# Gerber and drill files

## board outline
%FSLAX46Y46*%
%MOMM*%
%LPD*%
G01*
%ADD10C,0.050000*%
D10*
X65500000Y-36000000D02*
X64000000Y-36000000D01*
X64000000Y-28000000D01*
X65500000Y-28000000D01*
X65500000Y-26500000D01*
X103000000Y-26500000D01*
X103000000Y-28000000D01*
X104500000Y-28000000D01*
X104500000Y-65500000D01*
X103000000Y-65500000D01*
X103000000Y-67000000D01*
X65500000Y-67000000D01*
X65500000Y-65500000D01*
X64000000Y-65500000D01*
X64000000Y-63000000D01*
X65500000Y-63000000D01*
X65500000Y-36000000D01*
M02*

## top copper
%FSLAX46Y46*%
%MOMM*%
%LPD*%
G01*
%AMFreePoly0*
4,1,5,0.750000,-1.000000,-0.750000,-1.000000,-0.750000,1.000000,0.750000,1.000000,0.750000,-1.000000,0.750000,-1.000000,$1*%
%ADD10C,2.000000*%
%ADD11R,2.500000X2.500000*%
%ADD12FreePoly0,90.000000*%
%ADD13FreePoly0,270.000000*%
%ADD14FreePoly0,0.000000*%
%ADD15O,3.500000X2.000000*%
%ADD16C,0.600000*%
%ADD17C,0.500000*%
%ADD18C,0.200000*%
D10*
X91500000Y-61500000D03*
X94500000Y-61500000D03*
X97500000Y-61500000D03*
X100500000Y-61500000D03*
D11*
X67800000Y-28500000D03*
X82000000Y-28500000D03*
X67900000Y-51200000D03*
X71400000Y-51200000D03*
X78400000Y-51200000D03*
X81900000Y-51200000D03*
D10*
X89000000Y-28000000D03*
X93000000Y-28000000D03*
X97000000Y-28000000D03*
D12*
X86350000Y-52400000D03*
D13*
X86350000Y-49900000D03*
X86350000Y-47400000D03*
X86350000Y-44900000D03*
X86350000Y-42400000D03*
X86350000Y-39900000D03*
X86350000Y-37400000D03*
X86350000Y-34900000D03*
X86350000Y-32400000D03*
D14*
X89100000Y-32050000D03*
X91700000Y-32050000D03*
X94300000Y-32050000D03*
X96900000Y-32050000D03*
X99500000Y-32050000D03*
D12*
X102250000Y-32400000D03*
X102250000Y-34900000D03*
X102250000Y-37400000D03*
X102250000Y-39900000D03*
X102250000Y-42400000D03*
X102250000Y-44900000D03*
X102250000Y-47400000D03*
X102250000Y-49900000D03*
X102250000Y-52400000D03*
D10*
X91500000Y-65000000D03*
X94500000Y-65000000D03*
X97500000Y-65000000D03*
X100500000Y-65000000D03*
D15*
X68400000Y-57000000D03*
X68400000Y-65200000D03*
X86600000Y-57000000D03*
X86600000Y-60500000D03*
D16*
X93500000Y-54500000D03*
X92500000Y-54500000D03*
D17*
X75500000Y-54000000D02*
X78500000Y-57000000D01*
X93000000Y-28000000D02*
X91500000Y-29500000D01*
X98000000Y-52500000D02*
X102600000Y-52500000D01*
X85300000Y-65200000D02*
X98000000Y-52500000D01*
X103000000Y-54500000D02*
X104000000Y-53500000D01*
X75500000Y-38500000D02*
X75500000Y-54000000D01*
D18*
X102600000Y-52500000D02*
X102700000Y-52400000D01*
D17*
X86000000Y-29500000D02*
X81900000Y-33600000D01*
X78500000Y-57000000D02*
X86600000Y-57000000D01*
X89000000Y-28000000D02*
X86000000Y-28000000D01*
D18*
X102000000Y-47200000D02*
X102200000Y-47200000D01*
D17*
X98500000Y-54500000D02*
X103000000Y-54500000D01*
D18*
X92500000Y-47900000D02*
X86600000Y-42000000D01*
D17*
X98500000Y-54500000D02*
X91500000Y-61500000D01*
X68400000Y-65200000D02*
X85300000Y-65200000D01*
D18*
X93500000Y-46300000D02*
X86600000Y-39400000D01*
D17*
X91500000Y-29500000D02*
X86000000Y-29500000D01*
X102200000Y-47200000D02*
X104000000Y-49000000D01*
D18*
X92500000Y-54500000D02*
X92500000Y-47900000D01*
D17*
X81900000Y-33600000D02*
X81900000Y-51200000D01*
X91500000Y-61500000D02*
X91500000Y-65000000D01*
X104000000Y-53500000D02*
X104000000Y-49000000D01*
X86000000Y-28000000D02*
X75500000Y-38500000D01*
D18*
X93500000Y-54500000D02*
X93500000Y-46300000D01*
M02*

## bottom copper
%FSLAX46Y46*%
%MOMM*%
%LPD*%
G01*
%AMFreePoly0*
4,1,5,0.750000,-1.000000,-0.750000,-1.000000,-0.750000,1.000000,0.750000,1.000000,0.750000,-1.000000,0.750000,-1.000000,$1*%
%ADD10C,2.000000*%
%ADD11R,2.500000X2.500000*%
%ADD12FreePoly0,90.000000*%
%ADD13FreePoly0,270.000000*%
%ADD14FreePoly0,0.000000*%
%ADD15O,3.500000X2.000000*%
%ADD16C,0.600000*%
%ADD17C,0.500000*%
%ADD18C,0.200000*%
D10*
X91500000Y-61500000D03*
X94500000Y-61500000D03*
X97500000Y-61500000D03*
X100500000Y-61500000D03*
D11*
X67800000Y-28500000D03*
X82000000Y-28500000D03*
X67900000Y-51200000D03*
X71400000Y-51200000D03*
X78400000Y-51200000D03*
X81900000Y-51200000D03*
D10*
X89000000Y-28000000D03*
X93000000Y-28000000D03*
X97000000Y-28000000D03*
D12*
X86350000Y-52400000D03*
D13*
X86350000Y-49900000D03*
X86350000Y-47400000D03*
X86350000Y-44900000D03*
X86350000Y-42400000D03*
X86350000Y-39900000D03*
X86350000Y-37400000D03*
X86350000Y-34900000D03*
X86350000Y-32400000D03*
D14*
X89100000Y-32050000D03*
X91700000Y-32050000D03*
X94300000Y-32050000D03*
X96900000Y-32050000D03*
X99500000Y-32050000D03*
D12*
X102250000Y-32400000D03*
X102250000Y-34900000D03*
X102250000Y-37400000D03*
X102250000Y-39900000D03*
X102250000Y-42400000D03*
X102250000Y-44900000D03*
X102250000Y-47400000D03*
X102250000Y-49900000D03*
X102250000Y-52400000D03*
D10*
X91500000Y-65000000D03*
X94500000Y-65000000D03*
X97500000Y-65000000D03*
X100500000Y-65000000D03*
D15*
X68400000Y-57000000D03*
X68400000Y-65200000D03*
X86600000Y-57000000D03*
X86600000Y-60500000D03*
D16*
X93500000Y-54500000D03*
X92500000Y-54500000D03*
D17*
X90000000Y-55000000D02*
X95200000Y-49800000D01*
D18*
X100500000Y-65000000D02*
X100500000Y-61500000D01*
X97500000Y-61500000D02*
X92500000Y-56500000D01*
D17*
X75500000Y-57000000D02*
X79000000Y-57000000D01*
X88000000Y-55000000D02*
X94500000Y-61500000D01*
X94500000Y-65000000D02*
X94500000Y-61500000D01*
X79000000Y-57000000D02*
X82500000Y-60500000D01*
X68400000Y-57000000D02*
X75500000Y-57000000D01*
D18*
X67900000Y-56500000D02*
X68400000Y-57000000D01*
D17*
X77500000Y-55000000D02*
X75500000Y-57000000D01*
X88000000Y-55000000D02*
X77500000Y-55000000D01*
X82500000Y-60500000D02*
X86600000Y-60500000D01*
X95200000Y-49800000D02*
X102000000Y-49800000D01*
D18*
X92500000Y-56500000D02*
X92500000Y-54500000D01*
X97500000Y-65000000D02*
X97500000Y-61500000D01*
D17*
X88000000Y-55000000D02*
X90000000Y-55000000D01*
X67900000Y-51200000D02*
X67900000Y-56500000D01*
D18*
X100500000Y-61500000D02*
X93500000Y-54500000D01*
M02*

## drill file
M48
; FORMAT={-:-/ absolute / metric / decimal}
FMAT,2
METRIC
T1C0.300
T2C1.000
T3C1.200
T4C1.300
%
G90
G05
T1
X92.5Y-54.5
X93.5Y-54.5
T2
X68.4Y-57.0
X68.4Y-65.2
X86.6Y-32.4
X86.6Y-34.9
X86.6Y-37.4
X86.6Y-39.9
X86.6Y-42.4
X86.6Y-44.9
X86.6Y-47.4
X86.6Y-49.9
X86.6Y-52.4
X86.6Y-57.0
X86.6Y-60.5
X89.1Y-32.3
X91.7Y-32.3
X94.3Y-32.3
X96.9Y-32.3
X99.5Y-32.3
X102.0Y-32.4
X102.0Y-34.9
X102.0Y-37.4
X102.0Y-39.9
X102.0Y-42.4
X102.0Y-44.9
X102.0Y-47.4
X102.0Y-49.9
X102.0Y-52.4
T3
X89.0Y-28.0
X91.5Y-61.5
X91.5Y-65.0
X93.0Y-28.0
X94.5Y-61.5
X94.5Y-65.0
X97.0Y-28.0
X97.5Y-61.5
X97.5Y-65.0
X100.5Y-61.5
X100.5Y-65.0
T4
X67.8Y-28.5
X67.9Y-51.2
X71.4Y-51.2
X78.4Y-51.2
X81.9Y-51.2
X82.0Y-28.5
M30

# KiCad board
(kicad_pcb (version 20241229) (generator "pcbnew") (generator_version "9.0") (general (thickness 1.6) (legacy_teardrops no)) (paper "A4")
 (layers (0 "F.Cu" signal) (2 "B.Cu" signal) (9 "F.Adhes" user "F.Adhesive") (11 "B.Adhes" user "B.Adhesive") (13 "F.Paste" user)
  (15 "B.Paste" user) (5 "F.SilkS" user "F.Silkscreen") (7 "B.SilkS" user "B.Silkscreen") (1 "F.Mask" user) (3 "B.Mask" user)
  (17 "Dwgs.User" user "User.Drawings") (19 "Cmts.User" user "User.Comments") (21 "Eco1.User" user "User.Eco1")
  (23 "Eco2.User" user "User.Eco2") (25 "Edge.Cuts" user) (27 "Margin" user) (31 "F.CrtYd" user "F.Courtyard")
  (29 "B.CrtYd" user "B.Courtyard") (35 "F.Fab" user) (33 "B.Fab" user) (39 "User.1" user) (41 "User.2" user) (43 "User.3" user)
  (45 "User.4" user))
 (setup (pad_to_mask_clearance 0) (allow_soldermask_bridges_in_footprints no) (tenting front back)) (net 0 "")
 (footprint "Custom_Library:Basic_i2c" (layer "F.Cu") (at 96 61.5)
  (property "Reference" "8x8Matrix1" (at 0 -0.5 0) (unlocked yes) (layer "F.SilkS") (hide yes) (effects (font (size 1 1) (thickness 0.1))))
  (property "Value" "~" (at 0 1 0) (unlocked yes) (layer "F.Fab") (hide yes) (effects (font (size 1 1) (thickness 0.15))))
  (pad "1" thru_hole circle (at -4.5 0) (size 2 2) (drill 1.2) (layers "*.Cu" "*.Mask") (remove_unused_layers no))
  (pad "2" thru_hole circle (at -1.5 0) (size 2 2) (drill 1.2) (layers "*.Cu" "*.Mask") (remove_unused_layers no))
  (pad "3" thru_hole circle (at 1.5 0) (size 2 2) (drill 1.2) (layers "*.Cu" "*.Mask") (remove_unused_layers no))
  (pad "4" thru_hole circle (at 4.5 0) (size 2 2) (drill 1.2) (layers "*.Cu" "*.Mask") (remove_unused_layers no)))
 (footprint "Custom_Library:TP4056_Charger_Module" (layer "F.Cu") (at 74.9 41)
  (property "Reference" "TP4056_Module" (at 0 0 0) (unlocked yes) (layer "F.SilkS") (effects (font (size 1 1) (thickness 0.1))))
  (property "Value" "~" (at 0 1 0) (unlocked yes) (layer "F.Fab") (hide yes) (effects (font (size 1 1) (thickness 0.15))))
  (pad "1" thru_hole rect (at -7.1 -12.5) (size 2.5 2.5) (drill 1.3) (layers "*.Cu" "*.Mask") (remove_unused_layers no)
   (thermal_bridge_angle 45))
  (pad "2" thru_hole rect (at 7.1 -12.5) (size 2.5 2.5) (drill 1.3) (layers "*.Cu" "*.Mask") (remove_unused_layers no)
   (thermal_bridge_angle 45))
  (pad "3" thru_hole rect (at -7 10.2) (size 2.5 2.5) (drill 1.3) (layers "*.Cu" "*.Mask") (remove_unused_layers no)
   (thermal_bridge_angle 45))
  (pad "4" thru_hole rect (at -3.5 10.2) (size 2.5 2.5) (drill 1.3) (layers "*.Cu" "*.Mask") (remove_unused_layers no)
   (thermal_bridge_angle 45))
  (pad "5" thru_hole rect (at 3.5 10.2) (size 2.5 2.5) (drill 1.3) (layers "*.Cu" "*.Mask") (remove_unused_layers no)
   (thermal_bridge_angle 45))
  (pad "6" thru_hole rect (at 7 10.2) (size 2.5 2.5) (drill 1.3) (layers "*.Cu" "*.Mask") (remove_unused_layers no)
   (thermal_bridge_angle 45)))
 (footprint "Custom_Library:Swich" (layer "F.Cu") (at 93 28)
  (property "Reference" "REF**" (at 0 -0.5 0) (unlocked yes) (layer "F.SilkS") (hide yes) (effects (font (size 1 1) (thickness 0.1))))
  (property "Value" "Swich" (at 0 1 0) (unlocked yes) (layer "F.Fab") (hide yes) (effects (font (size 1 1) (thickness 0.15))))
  (pad "1" thru_hole circle (at -4 0) (size 2 2) (drill 1.2) (layers "*.Cu" "*.Mask") (remove_unused_layers no))
  (pad "2" thru_hole circle (at 0 0) (size 2 2) (drill 1.2) (layers "*.Cu" "*.Mask") (remove_unused_layers no))
  (pad "3" thru_hole circle (at 4 0) (size 2 2) (drill 1.2) (layers "*.Cu" "*.Mask") (remove_unused_layers no)))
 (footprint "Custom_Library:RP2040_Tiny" (layer "F.Cu") (at 94.3 42 90)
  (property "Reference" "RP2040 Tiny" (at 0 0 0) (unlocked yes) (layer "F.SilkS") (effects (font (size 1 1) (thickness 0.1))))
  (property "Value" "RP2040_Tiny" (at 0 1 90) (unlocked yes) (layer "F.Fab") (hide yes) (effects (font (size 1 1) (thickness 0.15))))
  (pad "1" thru_hole custom (at -10.4 -7.7 90) (size 1.5 2) (drill 1 (offset 0 -0.25)) (layers "*.Cu" "*.Mask") (remove_unused_layers no)
   (options (clearance outline) (anchor rect)) (primitives))
  (pad "2" thru_hole custom (at -7.9 -7.7 270) (size 1.5 2) (drill 1 (offset 0 0.25)) (layers "*.Cu" "*.Mask") (remove_unused_layers no)
   (options (clearance outline) (anchor rect)) (primitives))
  (pad "3" thru_hole custom (at -5.4 -7.7 270) (size 1.5 2) (drill 1 (offset 0 0.25)) (layers "*.Cu" "*.Mask") (remove_unused_layers no)
   (options (clearance outline) (anchor rect)) (primitives))
  (pad "4" thru_hole custom (at -2.9 -7.7 270) (size 1.5 2) (drill 1 (offset 0 0.25)) (layers "*.Cu" "*.Mask") (remove_unused_layers no)
   (options (clearance outline) (anchor rect)) (primitives))
  (pad "5" thru_hole custom (at -0.4 -7.7 270) (size 1.5 2) (drill 1 (offset 0 0.25)) (layers "*.Cu" "*.Mask") (remove_unused_layers no)
   (options (clearance outline) (anchor rect)) (primitives))
  (pad "6" thru_hole custom (at 2.1 -7.7 270) (size 1.5 2) (drill 1 (offset 0 0.25)) (layers "*.Cu" "*.Mask") (remove_unused_layers no)
   (options (clearance outline) (anchor rect)) (primitives))
  (pad "7" thru_hole custom (at 4.6 -7.7 270) (size 1.5 2) (drill 1 (offset 0 0.25)) (layers "*.Cu" "*.Mask") (remove_unused_layers no)
   (options (clearance outline) (anchor rect)) (primitives))
  (pad "8" thru_hole custom (at 7.1 -7.7 270) (size 1.5 2) (drill 1 (offset 0 0.25)) (layers "*.Cu" "*.Mask") (remove_unused_layers no)
   (options (clearance outline) (anchor rect)) (primitives))
  (pad "9" thru_hole custom (at 9.6 -7.7 270) (size 1.5 2) (drill 1 (offset 0 0.25)) (layers "*.Cu" "*.Mask") (remove_unused_layers no)
   (options (clearance outline) (anchor rect)) (primitives))
  (pad "10" thru_hole custom (at 9.7 -5.2) (size 1.5 2) (drill 1 (offset 0 -0.25)) (layers "*.Cu" "*.Mask") (remove_unused_layers no)
   (options (clearance outline) (anchor rect)) (primitives))
  (pad "11" thru_hole custom (at 9.7 -2.6) (size 1.5 2) (drill 1 (offset 0 -0.25)) (layers "*.Cu" "*.Mask") (remove_unused_layers no)
   (options (clearance outline) (anchor rect)) (primitives))
  (pad "12" thru_hole custom (at 9.7 0) (size 1.5 2) (drill 1 (offset 0 -0.25)) (layers "*.Cu" "*.Mask") (remove_unused_layers no)
   (options (clearance outline) (anchor rect)) (primitives))
  (pad "13" thru_hole custom (at 9.7 2.6) (size 1.5 2) (drill 1 (offset 0 -0.25)) (layers "*.Cu" "*.Mask") (remove_unused_layers no)
   (options (clearance outline) (anchor rect)) (primitives))
  (pad "14" thru_hole custom (at 9.7 5.2) (size 1.5 2) (drill 1 (offset 0 -0.25)) (layers "*.Cu" "*.Mask") (remove_unused_layers no)
   (options (clearance outline) (anchor rect)) (primitives))
  (pad "15" thru_hole custom (at 9.6 7.7 90) (size 1.5 2) (drill 1 (offset 0 0.25)) (layers "*.Cu" "*.Mask") (remove_unused_layers no)
   (options (clearance outline) (anchor rect)) (primitives))
  (pad "16" thru_hole custom (at 7.1 7.7 90) (size 1.5 2) (drill 1 (offset 0 0.25)) (layers "*.Cu" "*.Mask") (remove_unused_layers no)
   (options (clearance outline) (anchor rect)) (primitives))
  (pad "17" thru_hole custom (at 4.6 7.7 90) (size 1.5 2) (drill 1 (offset 0 0.25)) (layers "*.Cu" "*.Mask") (remove_unused_layers no)
   (options (clearance outline) (anchor rect)) (primitives))
  (pad "18" thru_hole custom (at 2.1 7.7 90) (size 1.5 2) (drill 1 (offset 0 0.25)) (layers "*.Cu" "*.Mask") (remove_unused_layers no)
   (options (clearance outline) (anchor rect)) (primitives))
  (pad "19" thru_hole custom (at -0.4 7.7 90) (size 1.5 2) (drill 1 (offset 0 0.25)) (layers "*.Cu" "*.Mask") (remove_unused_layers no)
   (options (clearance outline) (anchor rect)) (primitives))
  (pad "20" thru_hole custom (at -2.9 7.7 90) (size 1.5 2) (drill 1 (offset 0 0.25)) (layers "*.Cu" "*.Mask") (remove_unused_layers no)
   (options (clearance outline) (anchor rect)) (primitives))
  (pad "21" thru_hole custom (at -5.4 7.7 90) (size 1.5 2) (drill 1 (offset 0 0.25)) (layers "*.Cu" "*.Mask") (remove_unused_layers no)
   (options (clearance outline) (anchor rect)) (primitives))
  (pad "22" thru_hole custom (at -7.9 7.7 90) (size 1.5 2) (drill 1 (offset 0 0.25)) (layers "*.Cu" "*.Mask") (remove_unused_layers no)
   (options (clearance outline) (anchor rect)) (primitives))
  (pad "23" thru_hole custom (at -10.4 7.7 90) (size 1.5 2) (drill 1 (offset 0 0.25)) (layers "*.Cu" "*.Mask") (remove_unused_layers no)
   (options (clearance outline) (anchor rect)) (primitives))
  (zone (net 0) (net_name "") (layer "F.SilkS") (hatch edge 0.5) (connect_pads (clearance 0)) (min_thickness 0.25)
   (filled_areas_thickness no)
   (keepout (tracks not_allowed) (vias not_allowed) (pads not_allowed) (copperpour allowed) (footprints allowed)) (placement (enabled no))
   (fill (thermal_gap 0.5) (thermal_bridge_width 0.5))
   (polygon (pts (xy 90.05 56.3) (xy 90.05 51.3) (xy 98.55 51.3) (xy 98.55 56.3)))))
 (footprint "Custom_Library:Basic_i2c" (layer "F.Cu") (at 96 65)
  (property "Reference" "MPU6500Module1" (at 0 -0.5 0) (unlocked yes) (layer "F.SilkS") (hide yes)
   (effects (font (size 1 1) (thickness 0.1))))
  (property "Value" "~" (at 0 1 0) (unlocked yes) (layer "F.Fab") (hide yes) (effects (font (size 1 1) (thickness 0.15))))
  (pad "1" thru_hole circle (at -4.5 0) (size 2 2) (drill 1.2) (layers "*.Cu" "*.Mask") (remove_unused_layers no))
  (pad "2" thru_hole circle (at -1.5 0) (size 2 2) (drill 1.2) (layers "*.Cu" "*.Mask") (remove_unused_layers no))
  (pad "3" thru_hole circle (at 1.5 0) (size 2 2) (drill 1.2) (layers "*.Cu" "*.Mask") (remove_unused_layers no))
  (pad "4" thru_hole circle (at 4.5 0) (size 2 2) (drill 1.2) (layers "*.Cu" "*.Mask") (remove_unused_layers no)))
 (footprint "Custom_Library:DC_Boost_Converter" (layer "F.Cu") (at 77.5 61.1)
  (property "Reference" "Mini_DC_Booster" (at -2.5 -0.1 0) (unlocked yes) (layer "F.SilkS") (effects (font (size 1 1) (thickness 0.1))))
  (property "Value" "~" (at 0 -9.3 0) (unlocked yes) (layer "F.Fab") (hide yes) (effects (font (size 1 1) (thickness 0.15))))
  (pad "1" thru_hole oval (at -9.1 -4.1 90) (size 2 3.5) (drill 1) (layers "*.Cu" "*.Mask") (remove_unused_layers no)
   (thermal_bridge_angle 45))
  (pad "2" thru_hole oval (at -9.1 4.1 90) (size 2 3.5) (drill 1) (layers "*.Cu" "*.Mask") (remove_unused_layers no)
   (thermal_bridge_angle 45))
  (pad "3" thru_hole oval (at 9.1 -4.1 90) (size 2 3.5) (drill 1) (layers "*.Cu" "*.Mask") (remove_unused_layers no)
   (thermal_bridge_angle 45))
  (pad "4" thru_hole oval (at 9.1 -0.6 90) (size 2 3.5) (drill 1) (layers "*.Cu" "*.Mask") (remove_unused_layers no)
   (thermal_bridge_angle 45)))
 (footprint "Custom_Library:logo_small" (layer "F.Cu") (at 95.5 56)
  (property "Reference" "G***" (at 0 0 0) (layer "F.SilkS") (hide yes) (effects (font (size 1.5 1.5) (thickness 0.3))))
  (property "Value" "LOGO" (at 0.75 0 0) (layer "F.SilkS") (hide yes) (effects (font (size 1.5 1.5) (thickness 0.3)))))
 (gr_poly
  (pts (xy 65.5 36) (xy 64 36) (xy 64 28) (xy 65.5 28) (xy 65.5 26.5) (xy 103 26.5) (xy 103 28) (xy 104.5 28) (xy 104.5 65.5) (xy 103 65.5)
   (xy 103 67) (xy 65.5 67) (xy 65.5 65.5) (xy 64 65.5) (xy 64 63) (xy 65.5 63))
  (stroke (width 0.05) (type solid)) (fill no) (layer "Edge.Cuts"))
 (segment (start 75.5 54) (end 78.5 57) (width 0.5) (layer "F.Cu") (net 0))
 (segment (start 93 28) (end 91.5 29.5) (width 0.5) (layer "F.Cu") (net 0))
 (segment (start 98 52.5) (end 102.6 52.5) (width 0.5) (layer "F.Cu") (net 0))
 (segment (start 85.3 65.2) (end 98 52.5) (width 0.5) (layer "F.Cu") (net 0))
 (segment (start 103 54.5) (end 104 53.5) (width 0.5) (layer "F.Cu") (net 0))
 (segment (start 75.5 38.5) (end 75.5 54) (width 0.5) (layer "F.Cu") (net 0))
 (segment (start 102.6 52.5) (end 102.7 52.4) (width 0.2) (layer "F.Cu") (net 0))
 (segment (start 86 29.5) (end 81.9 33.6) (width 0.5) (layer "F.Cu") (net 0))
 (segment (start 78.5 57) (end 86.6 57) (width 0.5) (layer "F.Cu") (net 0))
 (segment (start 89 28) (end 86 28) (width 0.5) (layer "F.Cu") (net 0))
 (segment (start 102 47.2) (end 102.2 47.2) (width 0.2) (layer "F.Cu") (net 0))
 (segment (start 98.5 54.5) (end 103 54.5) (width 0.5) (layer "F.Cu") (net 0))
 (segment (start 92.5 47.9) (end 86.6 42) (width 0.2) (layer "F.Cu") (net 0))
 (segment (start 98.5 54.5) (end 91.5 61.5) (width 0.5) (layer "F.Cu") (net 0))
 (segment (start 68.4 65.2) (end 85.3 65.2) (width 0.5) (layer "F.Cu") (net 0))
 (segment (start 93.5 46.3) (end 86.6 39.4) (width 0.2) (layer "F.Cu") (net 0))
 (segment (start 91.5 29.5) (end 86 29.5) (width 0.5) (layer "F.Cu") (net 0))
 (segment (start 102.2 47.2) (end 104 49) (width 0.5) (layer "F.Cu") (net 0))
 (segment (start 92.5 54.5) (end 92.5 47.9) (width 0.2) (layer "F.Cu") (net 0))
 (segment (start 81.9 33.6) (end 81.9 51.2) (width 0.5) (layer "F.Cu") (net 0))
 (segment (start 91.5 61.5) (end 91.5 65) (width 0.5) (layer "F.Cu") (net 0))
 (segment (start 104 53.5) (end 104 49) (width 0.5) (layer "F.Cu") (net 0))
 (segment (start 86 28) (end 75.5 38.5) (width 0.5) (layer "F.Cu") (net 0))
 (segment (start 93.5 54.5) (end 93.5 46.3) (width 0.2) (layer "F.Cu") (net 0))
 (via (at 93.5 54.5) (size 0.6) (drill 0.3) (layers "F.Cu" "B.Cu") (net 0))
 (via (at 92.5 54.5) (size 0.6) (drill 0.3) (layers "F.Cu" "B.Cu") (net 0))
 (segment (start 90 55) (end 95.2 49.8) (width 0.5) (layer "B.Cu") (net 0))
 (segment (start 100.5 65) (end 100.5 61.5) (width 0.2) (layer "B.Cu") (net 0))
 (segment (start 97.5 61.5) (end 92.5 56.5) (width 0.2) (layer "B.Cu") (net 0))
 (segment (start 75.5 57) (end 79 57) (width 0.5) (layer "B.Cu") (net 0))
 (segment (start 88 55) (end 94.5 61.5) (width 0.5) (layer "B.Cu") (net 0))
 (segment (start 94.5 65) (end 94.5 61.5) (width 0.5) (layer "B.Cu") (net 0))
 (segment (start 79 57) (end 82.5 60.5) (width 0.5) (layer "B.Cu") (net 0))
 (segment (start 68.4 57) (end 75.5 57) (width 0.5) (layer "B.Cu") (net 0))
 (segment (start 67.9 56.5) (end 68.4 57) (width 0.2) (layer "B.Cu") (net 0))
 (segment (start 77.5 55) (end 75.5 57) (width 0.5) (layer "B.Cu") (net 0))
 (segment (start 88 55) (end 77.5 55) (width 0.5) (layer "B.Cu") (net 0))
 (segment (start 82.5 60.5) (end 86.6 60.5) (width 0.5) (layer "B.Cu") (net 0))
 (segment (start 95.2 49.8) (end 102 49.8) (width 0.5) (layer "B.Cu") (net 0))
 (segment (start 92.5 56.5) (end 92.5 54.5) (width 0.2) (layer "B.Cu") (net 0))
 (segment (start 97.5 65) (end 97.5 61.5) (width 0.2) (layer "B.Cu") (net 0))
 (segment (start 88 55) (end 90 55) (width 0.5) (layer "B.Cu") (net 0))
 (segment (start 67.9 51.2) (end 67.9 56.5) (width 0.5) (layer "B.Cu") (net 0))
 (segment (start 100.5 61.5) (end 93.5 54.5) (width 0.2) (layer "B.Cu") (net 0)))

